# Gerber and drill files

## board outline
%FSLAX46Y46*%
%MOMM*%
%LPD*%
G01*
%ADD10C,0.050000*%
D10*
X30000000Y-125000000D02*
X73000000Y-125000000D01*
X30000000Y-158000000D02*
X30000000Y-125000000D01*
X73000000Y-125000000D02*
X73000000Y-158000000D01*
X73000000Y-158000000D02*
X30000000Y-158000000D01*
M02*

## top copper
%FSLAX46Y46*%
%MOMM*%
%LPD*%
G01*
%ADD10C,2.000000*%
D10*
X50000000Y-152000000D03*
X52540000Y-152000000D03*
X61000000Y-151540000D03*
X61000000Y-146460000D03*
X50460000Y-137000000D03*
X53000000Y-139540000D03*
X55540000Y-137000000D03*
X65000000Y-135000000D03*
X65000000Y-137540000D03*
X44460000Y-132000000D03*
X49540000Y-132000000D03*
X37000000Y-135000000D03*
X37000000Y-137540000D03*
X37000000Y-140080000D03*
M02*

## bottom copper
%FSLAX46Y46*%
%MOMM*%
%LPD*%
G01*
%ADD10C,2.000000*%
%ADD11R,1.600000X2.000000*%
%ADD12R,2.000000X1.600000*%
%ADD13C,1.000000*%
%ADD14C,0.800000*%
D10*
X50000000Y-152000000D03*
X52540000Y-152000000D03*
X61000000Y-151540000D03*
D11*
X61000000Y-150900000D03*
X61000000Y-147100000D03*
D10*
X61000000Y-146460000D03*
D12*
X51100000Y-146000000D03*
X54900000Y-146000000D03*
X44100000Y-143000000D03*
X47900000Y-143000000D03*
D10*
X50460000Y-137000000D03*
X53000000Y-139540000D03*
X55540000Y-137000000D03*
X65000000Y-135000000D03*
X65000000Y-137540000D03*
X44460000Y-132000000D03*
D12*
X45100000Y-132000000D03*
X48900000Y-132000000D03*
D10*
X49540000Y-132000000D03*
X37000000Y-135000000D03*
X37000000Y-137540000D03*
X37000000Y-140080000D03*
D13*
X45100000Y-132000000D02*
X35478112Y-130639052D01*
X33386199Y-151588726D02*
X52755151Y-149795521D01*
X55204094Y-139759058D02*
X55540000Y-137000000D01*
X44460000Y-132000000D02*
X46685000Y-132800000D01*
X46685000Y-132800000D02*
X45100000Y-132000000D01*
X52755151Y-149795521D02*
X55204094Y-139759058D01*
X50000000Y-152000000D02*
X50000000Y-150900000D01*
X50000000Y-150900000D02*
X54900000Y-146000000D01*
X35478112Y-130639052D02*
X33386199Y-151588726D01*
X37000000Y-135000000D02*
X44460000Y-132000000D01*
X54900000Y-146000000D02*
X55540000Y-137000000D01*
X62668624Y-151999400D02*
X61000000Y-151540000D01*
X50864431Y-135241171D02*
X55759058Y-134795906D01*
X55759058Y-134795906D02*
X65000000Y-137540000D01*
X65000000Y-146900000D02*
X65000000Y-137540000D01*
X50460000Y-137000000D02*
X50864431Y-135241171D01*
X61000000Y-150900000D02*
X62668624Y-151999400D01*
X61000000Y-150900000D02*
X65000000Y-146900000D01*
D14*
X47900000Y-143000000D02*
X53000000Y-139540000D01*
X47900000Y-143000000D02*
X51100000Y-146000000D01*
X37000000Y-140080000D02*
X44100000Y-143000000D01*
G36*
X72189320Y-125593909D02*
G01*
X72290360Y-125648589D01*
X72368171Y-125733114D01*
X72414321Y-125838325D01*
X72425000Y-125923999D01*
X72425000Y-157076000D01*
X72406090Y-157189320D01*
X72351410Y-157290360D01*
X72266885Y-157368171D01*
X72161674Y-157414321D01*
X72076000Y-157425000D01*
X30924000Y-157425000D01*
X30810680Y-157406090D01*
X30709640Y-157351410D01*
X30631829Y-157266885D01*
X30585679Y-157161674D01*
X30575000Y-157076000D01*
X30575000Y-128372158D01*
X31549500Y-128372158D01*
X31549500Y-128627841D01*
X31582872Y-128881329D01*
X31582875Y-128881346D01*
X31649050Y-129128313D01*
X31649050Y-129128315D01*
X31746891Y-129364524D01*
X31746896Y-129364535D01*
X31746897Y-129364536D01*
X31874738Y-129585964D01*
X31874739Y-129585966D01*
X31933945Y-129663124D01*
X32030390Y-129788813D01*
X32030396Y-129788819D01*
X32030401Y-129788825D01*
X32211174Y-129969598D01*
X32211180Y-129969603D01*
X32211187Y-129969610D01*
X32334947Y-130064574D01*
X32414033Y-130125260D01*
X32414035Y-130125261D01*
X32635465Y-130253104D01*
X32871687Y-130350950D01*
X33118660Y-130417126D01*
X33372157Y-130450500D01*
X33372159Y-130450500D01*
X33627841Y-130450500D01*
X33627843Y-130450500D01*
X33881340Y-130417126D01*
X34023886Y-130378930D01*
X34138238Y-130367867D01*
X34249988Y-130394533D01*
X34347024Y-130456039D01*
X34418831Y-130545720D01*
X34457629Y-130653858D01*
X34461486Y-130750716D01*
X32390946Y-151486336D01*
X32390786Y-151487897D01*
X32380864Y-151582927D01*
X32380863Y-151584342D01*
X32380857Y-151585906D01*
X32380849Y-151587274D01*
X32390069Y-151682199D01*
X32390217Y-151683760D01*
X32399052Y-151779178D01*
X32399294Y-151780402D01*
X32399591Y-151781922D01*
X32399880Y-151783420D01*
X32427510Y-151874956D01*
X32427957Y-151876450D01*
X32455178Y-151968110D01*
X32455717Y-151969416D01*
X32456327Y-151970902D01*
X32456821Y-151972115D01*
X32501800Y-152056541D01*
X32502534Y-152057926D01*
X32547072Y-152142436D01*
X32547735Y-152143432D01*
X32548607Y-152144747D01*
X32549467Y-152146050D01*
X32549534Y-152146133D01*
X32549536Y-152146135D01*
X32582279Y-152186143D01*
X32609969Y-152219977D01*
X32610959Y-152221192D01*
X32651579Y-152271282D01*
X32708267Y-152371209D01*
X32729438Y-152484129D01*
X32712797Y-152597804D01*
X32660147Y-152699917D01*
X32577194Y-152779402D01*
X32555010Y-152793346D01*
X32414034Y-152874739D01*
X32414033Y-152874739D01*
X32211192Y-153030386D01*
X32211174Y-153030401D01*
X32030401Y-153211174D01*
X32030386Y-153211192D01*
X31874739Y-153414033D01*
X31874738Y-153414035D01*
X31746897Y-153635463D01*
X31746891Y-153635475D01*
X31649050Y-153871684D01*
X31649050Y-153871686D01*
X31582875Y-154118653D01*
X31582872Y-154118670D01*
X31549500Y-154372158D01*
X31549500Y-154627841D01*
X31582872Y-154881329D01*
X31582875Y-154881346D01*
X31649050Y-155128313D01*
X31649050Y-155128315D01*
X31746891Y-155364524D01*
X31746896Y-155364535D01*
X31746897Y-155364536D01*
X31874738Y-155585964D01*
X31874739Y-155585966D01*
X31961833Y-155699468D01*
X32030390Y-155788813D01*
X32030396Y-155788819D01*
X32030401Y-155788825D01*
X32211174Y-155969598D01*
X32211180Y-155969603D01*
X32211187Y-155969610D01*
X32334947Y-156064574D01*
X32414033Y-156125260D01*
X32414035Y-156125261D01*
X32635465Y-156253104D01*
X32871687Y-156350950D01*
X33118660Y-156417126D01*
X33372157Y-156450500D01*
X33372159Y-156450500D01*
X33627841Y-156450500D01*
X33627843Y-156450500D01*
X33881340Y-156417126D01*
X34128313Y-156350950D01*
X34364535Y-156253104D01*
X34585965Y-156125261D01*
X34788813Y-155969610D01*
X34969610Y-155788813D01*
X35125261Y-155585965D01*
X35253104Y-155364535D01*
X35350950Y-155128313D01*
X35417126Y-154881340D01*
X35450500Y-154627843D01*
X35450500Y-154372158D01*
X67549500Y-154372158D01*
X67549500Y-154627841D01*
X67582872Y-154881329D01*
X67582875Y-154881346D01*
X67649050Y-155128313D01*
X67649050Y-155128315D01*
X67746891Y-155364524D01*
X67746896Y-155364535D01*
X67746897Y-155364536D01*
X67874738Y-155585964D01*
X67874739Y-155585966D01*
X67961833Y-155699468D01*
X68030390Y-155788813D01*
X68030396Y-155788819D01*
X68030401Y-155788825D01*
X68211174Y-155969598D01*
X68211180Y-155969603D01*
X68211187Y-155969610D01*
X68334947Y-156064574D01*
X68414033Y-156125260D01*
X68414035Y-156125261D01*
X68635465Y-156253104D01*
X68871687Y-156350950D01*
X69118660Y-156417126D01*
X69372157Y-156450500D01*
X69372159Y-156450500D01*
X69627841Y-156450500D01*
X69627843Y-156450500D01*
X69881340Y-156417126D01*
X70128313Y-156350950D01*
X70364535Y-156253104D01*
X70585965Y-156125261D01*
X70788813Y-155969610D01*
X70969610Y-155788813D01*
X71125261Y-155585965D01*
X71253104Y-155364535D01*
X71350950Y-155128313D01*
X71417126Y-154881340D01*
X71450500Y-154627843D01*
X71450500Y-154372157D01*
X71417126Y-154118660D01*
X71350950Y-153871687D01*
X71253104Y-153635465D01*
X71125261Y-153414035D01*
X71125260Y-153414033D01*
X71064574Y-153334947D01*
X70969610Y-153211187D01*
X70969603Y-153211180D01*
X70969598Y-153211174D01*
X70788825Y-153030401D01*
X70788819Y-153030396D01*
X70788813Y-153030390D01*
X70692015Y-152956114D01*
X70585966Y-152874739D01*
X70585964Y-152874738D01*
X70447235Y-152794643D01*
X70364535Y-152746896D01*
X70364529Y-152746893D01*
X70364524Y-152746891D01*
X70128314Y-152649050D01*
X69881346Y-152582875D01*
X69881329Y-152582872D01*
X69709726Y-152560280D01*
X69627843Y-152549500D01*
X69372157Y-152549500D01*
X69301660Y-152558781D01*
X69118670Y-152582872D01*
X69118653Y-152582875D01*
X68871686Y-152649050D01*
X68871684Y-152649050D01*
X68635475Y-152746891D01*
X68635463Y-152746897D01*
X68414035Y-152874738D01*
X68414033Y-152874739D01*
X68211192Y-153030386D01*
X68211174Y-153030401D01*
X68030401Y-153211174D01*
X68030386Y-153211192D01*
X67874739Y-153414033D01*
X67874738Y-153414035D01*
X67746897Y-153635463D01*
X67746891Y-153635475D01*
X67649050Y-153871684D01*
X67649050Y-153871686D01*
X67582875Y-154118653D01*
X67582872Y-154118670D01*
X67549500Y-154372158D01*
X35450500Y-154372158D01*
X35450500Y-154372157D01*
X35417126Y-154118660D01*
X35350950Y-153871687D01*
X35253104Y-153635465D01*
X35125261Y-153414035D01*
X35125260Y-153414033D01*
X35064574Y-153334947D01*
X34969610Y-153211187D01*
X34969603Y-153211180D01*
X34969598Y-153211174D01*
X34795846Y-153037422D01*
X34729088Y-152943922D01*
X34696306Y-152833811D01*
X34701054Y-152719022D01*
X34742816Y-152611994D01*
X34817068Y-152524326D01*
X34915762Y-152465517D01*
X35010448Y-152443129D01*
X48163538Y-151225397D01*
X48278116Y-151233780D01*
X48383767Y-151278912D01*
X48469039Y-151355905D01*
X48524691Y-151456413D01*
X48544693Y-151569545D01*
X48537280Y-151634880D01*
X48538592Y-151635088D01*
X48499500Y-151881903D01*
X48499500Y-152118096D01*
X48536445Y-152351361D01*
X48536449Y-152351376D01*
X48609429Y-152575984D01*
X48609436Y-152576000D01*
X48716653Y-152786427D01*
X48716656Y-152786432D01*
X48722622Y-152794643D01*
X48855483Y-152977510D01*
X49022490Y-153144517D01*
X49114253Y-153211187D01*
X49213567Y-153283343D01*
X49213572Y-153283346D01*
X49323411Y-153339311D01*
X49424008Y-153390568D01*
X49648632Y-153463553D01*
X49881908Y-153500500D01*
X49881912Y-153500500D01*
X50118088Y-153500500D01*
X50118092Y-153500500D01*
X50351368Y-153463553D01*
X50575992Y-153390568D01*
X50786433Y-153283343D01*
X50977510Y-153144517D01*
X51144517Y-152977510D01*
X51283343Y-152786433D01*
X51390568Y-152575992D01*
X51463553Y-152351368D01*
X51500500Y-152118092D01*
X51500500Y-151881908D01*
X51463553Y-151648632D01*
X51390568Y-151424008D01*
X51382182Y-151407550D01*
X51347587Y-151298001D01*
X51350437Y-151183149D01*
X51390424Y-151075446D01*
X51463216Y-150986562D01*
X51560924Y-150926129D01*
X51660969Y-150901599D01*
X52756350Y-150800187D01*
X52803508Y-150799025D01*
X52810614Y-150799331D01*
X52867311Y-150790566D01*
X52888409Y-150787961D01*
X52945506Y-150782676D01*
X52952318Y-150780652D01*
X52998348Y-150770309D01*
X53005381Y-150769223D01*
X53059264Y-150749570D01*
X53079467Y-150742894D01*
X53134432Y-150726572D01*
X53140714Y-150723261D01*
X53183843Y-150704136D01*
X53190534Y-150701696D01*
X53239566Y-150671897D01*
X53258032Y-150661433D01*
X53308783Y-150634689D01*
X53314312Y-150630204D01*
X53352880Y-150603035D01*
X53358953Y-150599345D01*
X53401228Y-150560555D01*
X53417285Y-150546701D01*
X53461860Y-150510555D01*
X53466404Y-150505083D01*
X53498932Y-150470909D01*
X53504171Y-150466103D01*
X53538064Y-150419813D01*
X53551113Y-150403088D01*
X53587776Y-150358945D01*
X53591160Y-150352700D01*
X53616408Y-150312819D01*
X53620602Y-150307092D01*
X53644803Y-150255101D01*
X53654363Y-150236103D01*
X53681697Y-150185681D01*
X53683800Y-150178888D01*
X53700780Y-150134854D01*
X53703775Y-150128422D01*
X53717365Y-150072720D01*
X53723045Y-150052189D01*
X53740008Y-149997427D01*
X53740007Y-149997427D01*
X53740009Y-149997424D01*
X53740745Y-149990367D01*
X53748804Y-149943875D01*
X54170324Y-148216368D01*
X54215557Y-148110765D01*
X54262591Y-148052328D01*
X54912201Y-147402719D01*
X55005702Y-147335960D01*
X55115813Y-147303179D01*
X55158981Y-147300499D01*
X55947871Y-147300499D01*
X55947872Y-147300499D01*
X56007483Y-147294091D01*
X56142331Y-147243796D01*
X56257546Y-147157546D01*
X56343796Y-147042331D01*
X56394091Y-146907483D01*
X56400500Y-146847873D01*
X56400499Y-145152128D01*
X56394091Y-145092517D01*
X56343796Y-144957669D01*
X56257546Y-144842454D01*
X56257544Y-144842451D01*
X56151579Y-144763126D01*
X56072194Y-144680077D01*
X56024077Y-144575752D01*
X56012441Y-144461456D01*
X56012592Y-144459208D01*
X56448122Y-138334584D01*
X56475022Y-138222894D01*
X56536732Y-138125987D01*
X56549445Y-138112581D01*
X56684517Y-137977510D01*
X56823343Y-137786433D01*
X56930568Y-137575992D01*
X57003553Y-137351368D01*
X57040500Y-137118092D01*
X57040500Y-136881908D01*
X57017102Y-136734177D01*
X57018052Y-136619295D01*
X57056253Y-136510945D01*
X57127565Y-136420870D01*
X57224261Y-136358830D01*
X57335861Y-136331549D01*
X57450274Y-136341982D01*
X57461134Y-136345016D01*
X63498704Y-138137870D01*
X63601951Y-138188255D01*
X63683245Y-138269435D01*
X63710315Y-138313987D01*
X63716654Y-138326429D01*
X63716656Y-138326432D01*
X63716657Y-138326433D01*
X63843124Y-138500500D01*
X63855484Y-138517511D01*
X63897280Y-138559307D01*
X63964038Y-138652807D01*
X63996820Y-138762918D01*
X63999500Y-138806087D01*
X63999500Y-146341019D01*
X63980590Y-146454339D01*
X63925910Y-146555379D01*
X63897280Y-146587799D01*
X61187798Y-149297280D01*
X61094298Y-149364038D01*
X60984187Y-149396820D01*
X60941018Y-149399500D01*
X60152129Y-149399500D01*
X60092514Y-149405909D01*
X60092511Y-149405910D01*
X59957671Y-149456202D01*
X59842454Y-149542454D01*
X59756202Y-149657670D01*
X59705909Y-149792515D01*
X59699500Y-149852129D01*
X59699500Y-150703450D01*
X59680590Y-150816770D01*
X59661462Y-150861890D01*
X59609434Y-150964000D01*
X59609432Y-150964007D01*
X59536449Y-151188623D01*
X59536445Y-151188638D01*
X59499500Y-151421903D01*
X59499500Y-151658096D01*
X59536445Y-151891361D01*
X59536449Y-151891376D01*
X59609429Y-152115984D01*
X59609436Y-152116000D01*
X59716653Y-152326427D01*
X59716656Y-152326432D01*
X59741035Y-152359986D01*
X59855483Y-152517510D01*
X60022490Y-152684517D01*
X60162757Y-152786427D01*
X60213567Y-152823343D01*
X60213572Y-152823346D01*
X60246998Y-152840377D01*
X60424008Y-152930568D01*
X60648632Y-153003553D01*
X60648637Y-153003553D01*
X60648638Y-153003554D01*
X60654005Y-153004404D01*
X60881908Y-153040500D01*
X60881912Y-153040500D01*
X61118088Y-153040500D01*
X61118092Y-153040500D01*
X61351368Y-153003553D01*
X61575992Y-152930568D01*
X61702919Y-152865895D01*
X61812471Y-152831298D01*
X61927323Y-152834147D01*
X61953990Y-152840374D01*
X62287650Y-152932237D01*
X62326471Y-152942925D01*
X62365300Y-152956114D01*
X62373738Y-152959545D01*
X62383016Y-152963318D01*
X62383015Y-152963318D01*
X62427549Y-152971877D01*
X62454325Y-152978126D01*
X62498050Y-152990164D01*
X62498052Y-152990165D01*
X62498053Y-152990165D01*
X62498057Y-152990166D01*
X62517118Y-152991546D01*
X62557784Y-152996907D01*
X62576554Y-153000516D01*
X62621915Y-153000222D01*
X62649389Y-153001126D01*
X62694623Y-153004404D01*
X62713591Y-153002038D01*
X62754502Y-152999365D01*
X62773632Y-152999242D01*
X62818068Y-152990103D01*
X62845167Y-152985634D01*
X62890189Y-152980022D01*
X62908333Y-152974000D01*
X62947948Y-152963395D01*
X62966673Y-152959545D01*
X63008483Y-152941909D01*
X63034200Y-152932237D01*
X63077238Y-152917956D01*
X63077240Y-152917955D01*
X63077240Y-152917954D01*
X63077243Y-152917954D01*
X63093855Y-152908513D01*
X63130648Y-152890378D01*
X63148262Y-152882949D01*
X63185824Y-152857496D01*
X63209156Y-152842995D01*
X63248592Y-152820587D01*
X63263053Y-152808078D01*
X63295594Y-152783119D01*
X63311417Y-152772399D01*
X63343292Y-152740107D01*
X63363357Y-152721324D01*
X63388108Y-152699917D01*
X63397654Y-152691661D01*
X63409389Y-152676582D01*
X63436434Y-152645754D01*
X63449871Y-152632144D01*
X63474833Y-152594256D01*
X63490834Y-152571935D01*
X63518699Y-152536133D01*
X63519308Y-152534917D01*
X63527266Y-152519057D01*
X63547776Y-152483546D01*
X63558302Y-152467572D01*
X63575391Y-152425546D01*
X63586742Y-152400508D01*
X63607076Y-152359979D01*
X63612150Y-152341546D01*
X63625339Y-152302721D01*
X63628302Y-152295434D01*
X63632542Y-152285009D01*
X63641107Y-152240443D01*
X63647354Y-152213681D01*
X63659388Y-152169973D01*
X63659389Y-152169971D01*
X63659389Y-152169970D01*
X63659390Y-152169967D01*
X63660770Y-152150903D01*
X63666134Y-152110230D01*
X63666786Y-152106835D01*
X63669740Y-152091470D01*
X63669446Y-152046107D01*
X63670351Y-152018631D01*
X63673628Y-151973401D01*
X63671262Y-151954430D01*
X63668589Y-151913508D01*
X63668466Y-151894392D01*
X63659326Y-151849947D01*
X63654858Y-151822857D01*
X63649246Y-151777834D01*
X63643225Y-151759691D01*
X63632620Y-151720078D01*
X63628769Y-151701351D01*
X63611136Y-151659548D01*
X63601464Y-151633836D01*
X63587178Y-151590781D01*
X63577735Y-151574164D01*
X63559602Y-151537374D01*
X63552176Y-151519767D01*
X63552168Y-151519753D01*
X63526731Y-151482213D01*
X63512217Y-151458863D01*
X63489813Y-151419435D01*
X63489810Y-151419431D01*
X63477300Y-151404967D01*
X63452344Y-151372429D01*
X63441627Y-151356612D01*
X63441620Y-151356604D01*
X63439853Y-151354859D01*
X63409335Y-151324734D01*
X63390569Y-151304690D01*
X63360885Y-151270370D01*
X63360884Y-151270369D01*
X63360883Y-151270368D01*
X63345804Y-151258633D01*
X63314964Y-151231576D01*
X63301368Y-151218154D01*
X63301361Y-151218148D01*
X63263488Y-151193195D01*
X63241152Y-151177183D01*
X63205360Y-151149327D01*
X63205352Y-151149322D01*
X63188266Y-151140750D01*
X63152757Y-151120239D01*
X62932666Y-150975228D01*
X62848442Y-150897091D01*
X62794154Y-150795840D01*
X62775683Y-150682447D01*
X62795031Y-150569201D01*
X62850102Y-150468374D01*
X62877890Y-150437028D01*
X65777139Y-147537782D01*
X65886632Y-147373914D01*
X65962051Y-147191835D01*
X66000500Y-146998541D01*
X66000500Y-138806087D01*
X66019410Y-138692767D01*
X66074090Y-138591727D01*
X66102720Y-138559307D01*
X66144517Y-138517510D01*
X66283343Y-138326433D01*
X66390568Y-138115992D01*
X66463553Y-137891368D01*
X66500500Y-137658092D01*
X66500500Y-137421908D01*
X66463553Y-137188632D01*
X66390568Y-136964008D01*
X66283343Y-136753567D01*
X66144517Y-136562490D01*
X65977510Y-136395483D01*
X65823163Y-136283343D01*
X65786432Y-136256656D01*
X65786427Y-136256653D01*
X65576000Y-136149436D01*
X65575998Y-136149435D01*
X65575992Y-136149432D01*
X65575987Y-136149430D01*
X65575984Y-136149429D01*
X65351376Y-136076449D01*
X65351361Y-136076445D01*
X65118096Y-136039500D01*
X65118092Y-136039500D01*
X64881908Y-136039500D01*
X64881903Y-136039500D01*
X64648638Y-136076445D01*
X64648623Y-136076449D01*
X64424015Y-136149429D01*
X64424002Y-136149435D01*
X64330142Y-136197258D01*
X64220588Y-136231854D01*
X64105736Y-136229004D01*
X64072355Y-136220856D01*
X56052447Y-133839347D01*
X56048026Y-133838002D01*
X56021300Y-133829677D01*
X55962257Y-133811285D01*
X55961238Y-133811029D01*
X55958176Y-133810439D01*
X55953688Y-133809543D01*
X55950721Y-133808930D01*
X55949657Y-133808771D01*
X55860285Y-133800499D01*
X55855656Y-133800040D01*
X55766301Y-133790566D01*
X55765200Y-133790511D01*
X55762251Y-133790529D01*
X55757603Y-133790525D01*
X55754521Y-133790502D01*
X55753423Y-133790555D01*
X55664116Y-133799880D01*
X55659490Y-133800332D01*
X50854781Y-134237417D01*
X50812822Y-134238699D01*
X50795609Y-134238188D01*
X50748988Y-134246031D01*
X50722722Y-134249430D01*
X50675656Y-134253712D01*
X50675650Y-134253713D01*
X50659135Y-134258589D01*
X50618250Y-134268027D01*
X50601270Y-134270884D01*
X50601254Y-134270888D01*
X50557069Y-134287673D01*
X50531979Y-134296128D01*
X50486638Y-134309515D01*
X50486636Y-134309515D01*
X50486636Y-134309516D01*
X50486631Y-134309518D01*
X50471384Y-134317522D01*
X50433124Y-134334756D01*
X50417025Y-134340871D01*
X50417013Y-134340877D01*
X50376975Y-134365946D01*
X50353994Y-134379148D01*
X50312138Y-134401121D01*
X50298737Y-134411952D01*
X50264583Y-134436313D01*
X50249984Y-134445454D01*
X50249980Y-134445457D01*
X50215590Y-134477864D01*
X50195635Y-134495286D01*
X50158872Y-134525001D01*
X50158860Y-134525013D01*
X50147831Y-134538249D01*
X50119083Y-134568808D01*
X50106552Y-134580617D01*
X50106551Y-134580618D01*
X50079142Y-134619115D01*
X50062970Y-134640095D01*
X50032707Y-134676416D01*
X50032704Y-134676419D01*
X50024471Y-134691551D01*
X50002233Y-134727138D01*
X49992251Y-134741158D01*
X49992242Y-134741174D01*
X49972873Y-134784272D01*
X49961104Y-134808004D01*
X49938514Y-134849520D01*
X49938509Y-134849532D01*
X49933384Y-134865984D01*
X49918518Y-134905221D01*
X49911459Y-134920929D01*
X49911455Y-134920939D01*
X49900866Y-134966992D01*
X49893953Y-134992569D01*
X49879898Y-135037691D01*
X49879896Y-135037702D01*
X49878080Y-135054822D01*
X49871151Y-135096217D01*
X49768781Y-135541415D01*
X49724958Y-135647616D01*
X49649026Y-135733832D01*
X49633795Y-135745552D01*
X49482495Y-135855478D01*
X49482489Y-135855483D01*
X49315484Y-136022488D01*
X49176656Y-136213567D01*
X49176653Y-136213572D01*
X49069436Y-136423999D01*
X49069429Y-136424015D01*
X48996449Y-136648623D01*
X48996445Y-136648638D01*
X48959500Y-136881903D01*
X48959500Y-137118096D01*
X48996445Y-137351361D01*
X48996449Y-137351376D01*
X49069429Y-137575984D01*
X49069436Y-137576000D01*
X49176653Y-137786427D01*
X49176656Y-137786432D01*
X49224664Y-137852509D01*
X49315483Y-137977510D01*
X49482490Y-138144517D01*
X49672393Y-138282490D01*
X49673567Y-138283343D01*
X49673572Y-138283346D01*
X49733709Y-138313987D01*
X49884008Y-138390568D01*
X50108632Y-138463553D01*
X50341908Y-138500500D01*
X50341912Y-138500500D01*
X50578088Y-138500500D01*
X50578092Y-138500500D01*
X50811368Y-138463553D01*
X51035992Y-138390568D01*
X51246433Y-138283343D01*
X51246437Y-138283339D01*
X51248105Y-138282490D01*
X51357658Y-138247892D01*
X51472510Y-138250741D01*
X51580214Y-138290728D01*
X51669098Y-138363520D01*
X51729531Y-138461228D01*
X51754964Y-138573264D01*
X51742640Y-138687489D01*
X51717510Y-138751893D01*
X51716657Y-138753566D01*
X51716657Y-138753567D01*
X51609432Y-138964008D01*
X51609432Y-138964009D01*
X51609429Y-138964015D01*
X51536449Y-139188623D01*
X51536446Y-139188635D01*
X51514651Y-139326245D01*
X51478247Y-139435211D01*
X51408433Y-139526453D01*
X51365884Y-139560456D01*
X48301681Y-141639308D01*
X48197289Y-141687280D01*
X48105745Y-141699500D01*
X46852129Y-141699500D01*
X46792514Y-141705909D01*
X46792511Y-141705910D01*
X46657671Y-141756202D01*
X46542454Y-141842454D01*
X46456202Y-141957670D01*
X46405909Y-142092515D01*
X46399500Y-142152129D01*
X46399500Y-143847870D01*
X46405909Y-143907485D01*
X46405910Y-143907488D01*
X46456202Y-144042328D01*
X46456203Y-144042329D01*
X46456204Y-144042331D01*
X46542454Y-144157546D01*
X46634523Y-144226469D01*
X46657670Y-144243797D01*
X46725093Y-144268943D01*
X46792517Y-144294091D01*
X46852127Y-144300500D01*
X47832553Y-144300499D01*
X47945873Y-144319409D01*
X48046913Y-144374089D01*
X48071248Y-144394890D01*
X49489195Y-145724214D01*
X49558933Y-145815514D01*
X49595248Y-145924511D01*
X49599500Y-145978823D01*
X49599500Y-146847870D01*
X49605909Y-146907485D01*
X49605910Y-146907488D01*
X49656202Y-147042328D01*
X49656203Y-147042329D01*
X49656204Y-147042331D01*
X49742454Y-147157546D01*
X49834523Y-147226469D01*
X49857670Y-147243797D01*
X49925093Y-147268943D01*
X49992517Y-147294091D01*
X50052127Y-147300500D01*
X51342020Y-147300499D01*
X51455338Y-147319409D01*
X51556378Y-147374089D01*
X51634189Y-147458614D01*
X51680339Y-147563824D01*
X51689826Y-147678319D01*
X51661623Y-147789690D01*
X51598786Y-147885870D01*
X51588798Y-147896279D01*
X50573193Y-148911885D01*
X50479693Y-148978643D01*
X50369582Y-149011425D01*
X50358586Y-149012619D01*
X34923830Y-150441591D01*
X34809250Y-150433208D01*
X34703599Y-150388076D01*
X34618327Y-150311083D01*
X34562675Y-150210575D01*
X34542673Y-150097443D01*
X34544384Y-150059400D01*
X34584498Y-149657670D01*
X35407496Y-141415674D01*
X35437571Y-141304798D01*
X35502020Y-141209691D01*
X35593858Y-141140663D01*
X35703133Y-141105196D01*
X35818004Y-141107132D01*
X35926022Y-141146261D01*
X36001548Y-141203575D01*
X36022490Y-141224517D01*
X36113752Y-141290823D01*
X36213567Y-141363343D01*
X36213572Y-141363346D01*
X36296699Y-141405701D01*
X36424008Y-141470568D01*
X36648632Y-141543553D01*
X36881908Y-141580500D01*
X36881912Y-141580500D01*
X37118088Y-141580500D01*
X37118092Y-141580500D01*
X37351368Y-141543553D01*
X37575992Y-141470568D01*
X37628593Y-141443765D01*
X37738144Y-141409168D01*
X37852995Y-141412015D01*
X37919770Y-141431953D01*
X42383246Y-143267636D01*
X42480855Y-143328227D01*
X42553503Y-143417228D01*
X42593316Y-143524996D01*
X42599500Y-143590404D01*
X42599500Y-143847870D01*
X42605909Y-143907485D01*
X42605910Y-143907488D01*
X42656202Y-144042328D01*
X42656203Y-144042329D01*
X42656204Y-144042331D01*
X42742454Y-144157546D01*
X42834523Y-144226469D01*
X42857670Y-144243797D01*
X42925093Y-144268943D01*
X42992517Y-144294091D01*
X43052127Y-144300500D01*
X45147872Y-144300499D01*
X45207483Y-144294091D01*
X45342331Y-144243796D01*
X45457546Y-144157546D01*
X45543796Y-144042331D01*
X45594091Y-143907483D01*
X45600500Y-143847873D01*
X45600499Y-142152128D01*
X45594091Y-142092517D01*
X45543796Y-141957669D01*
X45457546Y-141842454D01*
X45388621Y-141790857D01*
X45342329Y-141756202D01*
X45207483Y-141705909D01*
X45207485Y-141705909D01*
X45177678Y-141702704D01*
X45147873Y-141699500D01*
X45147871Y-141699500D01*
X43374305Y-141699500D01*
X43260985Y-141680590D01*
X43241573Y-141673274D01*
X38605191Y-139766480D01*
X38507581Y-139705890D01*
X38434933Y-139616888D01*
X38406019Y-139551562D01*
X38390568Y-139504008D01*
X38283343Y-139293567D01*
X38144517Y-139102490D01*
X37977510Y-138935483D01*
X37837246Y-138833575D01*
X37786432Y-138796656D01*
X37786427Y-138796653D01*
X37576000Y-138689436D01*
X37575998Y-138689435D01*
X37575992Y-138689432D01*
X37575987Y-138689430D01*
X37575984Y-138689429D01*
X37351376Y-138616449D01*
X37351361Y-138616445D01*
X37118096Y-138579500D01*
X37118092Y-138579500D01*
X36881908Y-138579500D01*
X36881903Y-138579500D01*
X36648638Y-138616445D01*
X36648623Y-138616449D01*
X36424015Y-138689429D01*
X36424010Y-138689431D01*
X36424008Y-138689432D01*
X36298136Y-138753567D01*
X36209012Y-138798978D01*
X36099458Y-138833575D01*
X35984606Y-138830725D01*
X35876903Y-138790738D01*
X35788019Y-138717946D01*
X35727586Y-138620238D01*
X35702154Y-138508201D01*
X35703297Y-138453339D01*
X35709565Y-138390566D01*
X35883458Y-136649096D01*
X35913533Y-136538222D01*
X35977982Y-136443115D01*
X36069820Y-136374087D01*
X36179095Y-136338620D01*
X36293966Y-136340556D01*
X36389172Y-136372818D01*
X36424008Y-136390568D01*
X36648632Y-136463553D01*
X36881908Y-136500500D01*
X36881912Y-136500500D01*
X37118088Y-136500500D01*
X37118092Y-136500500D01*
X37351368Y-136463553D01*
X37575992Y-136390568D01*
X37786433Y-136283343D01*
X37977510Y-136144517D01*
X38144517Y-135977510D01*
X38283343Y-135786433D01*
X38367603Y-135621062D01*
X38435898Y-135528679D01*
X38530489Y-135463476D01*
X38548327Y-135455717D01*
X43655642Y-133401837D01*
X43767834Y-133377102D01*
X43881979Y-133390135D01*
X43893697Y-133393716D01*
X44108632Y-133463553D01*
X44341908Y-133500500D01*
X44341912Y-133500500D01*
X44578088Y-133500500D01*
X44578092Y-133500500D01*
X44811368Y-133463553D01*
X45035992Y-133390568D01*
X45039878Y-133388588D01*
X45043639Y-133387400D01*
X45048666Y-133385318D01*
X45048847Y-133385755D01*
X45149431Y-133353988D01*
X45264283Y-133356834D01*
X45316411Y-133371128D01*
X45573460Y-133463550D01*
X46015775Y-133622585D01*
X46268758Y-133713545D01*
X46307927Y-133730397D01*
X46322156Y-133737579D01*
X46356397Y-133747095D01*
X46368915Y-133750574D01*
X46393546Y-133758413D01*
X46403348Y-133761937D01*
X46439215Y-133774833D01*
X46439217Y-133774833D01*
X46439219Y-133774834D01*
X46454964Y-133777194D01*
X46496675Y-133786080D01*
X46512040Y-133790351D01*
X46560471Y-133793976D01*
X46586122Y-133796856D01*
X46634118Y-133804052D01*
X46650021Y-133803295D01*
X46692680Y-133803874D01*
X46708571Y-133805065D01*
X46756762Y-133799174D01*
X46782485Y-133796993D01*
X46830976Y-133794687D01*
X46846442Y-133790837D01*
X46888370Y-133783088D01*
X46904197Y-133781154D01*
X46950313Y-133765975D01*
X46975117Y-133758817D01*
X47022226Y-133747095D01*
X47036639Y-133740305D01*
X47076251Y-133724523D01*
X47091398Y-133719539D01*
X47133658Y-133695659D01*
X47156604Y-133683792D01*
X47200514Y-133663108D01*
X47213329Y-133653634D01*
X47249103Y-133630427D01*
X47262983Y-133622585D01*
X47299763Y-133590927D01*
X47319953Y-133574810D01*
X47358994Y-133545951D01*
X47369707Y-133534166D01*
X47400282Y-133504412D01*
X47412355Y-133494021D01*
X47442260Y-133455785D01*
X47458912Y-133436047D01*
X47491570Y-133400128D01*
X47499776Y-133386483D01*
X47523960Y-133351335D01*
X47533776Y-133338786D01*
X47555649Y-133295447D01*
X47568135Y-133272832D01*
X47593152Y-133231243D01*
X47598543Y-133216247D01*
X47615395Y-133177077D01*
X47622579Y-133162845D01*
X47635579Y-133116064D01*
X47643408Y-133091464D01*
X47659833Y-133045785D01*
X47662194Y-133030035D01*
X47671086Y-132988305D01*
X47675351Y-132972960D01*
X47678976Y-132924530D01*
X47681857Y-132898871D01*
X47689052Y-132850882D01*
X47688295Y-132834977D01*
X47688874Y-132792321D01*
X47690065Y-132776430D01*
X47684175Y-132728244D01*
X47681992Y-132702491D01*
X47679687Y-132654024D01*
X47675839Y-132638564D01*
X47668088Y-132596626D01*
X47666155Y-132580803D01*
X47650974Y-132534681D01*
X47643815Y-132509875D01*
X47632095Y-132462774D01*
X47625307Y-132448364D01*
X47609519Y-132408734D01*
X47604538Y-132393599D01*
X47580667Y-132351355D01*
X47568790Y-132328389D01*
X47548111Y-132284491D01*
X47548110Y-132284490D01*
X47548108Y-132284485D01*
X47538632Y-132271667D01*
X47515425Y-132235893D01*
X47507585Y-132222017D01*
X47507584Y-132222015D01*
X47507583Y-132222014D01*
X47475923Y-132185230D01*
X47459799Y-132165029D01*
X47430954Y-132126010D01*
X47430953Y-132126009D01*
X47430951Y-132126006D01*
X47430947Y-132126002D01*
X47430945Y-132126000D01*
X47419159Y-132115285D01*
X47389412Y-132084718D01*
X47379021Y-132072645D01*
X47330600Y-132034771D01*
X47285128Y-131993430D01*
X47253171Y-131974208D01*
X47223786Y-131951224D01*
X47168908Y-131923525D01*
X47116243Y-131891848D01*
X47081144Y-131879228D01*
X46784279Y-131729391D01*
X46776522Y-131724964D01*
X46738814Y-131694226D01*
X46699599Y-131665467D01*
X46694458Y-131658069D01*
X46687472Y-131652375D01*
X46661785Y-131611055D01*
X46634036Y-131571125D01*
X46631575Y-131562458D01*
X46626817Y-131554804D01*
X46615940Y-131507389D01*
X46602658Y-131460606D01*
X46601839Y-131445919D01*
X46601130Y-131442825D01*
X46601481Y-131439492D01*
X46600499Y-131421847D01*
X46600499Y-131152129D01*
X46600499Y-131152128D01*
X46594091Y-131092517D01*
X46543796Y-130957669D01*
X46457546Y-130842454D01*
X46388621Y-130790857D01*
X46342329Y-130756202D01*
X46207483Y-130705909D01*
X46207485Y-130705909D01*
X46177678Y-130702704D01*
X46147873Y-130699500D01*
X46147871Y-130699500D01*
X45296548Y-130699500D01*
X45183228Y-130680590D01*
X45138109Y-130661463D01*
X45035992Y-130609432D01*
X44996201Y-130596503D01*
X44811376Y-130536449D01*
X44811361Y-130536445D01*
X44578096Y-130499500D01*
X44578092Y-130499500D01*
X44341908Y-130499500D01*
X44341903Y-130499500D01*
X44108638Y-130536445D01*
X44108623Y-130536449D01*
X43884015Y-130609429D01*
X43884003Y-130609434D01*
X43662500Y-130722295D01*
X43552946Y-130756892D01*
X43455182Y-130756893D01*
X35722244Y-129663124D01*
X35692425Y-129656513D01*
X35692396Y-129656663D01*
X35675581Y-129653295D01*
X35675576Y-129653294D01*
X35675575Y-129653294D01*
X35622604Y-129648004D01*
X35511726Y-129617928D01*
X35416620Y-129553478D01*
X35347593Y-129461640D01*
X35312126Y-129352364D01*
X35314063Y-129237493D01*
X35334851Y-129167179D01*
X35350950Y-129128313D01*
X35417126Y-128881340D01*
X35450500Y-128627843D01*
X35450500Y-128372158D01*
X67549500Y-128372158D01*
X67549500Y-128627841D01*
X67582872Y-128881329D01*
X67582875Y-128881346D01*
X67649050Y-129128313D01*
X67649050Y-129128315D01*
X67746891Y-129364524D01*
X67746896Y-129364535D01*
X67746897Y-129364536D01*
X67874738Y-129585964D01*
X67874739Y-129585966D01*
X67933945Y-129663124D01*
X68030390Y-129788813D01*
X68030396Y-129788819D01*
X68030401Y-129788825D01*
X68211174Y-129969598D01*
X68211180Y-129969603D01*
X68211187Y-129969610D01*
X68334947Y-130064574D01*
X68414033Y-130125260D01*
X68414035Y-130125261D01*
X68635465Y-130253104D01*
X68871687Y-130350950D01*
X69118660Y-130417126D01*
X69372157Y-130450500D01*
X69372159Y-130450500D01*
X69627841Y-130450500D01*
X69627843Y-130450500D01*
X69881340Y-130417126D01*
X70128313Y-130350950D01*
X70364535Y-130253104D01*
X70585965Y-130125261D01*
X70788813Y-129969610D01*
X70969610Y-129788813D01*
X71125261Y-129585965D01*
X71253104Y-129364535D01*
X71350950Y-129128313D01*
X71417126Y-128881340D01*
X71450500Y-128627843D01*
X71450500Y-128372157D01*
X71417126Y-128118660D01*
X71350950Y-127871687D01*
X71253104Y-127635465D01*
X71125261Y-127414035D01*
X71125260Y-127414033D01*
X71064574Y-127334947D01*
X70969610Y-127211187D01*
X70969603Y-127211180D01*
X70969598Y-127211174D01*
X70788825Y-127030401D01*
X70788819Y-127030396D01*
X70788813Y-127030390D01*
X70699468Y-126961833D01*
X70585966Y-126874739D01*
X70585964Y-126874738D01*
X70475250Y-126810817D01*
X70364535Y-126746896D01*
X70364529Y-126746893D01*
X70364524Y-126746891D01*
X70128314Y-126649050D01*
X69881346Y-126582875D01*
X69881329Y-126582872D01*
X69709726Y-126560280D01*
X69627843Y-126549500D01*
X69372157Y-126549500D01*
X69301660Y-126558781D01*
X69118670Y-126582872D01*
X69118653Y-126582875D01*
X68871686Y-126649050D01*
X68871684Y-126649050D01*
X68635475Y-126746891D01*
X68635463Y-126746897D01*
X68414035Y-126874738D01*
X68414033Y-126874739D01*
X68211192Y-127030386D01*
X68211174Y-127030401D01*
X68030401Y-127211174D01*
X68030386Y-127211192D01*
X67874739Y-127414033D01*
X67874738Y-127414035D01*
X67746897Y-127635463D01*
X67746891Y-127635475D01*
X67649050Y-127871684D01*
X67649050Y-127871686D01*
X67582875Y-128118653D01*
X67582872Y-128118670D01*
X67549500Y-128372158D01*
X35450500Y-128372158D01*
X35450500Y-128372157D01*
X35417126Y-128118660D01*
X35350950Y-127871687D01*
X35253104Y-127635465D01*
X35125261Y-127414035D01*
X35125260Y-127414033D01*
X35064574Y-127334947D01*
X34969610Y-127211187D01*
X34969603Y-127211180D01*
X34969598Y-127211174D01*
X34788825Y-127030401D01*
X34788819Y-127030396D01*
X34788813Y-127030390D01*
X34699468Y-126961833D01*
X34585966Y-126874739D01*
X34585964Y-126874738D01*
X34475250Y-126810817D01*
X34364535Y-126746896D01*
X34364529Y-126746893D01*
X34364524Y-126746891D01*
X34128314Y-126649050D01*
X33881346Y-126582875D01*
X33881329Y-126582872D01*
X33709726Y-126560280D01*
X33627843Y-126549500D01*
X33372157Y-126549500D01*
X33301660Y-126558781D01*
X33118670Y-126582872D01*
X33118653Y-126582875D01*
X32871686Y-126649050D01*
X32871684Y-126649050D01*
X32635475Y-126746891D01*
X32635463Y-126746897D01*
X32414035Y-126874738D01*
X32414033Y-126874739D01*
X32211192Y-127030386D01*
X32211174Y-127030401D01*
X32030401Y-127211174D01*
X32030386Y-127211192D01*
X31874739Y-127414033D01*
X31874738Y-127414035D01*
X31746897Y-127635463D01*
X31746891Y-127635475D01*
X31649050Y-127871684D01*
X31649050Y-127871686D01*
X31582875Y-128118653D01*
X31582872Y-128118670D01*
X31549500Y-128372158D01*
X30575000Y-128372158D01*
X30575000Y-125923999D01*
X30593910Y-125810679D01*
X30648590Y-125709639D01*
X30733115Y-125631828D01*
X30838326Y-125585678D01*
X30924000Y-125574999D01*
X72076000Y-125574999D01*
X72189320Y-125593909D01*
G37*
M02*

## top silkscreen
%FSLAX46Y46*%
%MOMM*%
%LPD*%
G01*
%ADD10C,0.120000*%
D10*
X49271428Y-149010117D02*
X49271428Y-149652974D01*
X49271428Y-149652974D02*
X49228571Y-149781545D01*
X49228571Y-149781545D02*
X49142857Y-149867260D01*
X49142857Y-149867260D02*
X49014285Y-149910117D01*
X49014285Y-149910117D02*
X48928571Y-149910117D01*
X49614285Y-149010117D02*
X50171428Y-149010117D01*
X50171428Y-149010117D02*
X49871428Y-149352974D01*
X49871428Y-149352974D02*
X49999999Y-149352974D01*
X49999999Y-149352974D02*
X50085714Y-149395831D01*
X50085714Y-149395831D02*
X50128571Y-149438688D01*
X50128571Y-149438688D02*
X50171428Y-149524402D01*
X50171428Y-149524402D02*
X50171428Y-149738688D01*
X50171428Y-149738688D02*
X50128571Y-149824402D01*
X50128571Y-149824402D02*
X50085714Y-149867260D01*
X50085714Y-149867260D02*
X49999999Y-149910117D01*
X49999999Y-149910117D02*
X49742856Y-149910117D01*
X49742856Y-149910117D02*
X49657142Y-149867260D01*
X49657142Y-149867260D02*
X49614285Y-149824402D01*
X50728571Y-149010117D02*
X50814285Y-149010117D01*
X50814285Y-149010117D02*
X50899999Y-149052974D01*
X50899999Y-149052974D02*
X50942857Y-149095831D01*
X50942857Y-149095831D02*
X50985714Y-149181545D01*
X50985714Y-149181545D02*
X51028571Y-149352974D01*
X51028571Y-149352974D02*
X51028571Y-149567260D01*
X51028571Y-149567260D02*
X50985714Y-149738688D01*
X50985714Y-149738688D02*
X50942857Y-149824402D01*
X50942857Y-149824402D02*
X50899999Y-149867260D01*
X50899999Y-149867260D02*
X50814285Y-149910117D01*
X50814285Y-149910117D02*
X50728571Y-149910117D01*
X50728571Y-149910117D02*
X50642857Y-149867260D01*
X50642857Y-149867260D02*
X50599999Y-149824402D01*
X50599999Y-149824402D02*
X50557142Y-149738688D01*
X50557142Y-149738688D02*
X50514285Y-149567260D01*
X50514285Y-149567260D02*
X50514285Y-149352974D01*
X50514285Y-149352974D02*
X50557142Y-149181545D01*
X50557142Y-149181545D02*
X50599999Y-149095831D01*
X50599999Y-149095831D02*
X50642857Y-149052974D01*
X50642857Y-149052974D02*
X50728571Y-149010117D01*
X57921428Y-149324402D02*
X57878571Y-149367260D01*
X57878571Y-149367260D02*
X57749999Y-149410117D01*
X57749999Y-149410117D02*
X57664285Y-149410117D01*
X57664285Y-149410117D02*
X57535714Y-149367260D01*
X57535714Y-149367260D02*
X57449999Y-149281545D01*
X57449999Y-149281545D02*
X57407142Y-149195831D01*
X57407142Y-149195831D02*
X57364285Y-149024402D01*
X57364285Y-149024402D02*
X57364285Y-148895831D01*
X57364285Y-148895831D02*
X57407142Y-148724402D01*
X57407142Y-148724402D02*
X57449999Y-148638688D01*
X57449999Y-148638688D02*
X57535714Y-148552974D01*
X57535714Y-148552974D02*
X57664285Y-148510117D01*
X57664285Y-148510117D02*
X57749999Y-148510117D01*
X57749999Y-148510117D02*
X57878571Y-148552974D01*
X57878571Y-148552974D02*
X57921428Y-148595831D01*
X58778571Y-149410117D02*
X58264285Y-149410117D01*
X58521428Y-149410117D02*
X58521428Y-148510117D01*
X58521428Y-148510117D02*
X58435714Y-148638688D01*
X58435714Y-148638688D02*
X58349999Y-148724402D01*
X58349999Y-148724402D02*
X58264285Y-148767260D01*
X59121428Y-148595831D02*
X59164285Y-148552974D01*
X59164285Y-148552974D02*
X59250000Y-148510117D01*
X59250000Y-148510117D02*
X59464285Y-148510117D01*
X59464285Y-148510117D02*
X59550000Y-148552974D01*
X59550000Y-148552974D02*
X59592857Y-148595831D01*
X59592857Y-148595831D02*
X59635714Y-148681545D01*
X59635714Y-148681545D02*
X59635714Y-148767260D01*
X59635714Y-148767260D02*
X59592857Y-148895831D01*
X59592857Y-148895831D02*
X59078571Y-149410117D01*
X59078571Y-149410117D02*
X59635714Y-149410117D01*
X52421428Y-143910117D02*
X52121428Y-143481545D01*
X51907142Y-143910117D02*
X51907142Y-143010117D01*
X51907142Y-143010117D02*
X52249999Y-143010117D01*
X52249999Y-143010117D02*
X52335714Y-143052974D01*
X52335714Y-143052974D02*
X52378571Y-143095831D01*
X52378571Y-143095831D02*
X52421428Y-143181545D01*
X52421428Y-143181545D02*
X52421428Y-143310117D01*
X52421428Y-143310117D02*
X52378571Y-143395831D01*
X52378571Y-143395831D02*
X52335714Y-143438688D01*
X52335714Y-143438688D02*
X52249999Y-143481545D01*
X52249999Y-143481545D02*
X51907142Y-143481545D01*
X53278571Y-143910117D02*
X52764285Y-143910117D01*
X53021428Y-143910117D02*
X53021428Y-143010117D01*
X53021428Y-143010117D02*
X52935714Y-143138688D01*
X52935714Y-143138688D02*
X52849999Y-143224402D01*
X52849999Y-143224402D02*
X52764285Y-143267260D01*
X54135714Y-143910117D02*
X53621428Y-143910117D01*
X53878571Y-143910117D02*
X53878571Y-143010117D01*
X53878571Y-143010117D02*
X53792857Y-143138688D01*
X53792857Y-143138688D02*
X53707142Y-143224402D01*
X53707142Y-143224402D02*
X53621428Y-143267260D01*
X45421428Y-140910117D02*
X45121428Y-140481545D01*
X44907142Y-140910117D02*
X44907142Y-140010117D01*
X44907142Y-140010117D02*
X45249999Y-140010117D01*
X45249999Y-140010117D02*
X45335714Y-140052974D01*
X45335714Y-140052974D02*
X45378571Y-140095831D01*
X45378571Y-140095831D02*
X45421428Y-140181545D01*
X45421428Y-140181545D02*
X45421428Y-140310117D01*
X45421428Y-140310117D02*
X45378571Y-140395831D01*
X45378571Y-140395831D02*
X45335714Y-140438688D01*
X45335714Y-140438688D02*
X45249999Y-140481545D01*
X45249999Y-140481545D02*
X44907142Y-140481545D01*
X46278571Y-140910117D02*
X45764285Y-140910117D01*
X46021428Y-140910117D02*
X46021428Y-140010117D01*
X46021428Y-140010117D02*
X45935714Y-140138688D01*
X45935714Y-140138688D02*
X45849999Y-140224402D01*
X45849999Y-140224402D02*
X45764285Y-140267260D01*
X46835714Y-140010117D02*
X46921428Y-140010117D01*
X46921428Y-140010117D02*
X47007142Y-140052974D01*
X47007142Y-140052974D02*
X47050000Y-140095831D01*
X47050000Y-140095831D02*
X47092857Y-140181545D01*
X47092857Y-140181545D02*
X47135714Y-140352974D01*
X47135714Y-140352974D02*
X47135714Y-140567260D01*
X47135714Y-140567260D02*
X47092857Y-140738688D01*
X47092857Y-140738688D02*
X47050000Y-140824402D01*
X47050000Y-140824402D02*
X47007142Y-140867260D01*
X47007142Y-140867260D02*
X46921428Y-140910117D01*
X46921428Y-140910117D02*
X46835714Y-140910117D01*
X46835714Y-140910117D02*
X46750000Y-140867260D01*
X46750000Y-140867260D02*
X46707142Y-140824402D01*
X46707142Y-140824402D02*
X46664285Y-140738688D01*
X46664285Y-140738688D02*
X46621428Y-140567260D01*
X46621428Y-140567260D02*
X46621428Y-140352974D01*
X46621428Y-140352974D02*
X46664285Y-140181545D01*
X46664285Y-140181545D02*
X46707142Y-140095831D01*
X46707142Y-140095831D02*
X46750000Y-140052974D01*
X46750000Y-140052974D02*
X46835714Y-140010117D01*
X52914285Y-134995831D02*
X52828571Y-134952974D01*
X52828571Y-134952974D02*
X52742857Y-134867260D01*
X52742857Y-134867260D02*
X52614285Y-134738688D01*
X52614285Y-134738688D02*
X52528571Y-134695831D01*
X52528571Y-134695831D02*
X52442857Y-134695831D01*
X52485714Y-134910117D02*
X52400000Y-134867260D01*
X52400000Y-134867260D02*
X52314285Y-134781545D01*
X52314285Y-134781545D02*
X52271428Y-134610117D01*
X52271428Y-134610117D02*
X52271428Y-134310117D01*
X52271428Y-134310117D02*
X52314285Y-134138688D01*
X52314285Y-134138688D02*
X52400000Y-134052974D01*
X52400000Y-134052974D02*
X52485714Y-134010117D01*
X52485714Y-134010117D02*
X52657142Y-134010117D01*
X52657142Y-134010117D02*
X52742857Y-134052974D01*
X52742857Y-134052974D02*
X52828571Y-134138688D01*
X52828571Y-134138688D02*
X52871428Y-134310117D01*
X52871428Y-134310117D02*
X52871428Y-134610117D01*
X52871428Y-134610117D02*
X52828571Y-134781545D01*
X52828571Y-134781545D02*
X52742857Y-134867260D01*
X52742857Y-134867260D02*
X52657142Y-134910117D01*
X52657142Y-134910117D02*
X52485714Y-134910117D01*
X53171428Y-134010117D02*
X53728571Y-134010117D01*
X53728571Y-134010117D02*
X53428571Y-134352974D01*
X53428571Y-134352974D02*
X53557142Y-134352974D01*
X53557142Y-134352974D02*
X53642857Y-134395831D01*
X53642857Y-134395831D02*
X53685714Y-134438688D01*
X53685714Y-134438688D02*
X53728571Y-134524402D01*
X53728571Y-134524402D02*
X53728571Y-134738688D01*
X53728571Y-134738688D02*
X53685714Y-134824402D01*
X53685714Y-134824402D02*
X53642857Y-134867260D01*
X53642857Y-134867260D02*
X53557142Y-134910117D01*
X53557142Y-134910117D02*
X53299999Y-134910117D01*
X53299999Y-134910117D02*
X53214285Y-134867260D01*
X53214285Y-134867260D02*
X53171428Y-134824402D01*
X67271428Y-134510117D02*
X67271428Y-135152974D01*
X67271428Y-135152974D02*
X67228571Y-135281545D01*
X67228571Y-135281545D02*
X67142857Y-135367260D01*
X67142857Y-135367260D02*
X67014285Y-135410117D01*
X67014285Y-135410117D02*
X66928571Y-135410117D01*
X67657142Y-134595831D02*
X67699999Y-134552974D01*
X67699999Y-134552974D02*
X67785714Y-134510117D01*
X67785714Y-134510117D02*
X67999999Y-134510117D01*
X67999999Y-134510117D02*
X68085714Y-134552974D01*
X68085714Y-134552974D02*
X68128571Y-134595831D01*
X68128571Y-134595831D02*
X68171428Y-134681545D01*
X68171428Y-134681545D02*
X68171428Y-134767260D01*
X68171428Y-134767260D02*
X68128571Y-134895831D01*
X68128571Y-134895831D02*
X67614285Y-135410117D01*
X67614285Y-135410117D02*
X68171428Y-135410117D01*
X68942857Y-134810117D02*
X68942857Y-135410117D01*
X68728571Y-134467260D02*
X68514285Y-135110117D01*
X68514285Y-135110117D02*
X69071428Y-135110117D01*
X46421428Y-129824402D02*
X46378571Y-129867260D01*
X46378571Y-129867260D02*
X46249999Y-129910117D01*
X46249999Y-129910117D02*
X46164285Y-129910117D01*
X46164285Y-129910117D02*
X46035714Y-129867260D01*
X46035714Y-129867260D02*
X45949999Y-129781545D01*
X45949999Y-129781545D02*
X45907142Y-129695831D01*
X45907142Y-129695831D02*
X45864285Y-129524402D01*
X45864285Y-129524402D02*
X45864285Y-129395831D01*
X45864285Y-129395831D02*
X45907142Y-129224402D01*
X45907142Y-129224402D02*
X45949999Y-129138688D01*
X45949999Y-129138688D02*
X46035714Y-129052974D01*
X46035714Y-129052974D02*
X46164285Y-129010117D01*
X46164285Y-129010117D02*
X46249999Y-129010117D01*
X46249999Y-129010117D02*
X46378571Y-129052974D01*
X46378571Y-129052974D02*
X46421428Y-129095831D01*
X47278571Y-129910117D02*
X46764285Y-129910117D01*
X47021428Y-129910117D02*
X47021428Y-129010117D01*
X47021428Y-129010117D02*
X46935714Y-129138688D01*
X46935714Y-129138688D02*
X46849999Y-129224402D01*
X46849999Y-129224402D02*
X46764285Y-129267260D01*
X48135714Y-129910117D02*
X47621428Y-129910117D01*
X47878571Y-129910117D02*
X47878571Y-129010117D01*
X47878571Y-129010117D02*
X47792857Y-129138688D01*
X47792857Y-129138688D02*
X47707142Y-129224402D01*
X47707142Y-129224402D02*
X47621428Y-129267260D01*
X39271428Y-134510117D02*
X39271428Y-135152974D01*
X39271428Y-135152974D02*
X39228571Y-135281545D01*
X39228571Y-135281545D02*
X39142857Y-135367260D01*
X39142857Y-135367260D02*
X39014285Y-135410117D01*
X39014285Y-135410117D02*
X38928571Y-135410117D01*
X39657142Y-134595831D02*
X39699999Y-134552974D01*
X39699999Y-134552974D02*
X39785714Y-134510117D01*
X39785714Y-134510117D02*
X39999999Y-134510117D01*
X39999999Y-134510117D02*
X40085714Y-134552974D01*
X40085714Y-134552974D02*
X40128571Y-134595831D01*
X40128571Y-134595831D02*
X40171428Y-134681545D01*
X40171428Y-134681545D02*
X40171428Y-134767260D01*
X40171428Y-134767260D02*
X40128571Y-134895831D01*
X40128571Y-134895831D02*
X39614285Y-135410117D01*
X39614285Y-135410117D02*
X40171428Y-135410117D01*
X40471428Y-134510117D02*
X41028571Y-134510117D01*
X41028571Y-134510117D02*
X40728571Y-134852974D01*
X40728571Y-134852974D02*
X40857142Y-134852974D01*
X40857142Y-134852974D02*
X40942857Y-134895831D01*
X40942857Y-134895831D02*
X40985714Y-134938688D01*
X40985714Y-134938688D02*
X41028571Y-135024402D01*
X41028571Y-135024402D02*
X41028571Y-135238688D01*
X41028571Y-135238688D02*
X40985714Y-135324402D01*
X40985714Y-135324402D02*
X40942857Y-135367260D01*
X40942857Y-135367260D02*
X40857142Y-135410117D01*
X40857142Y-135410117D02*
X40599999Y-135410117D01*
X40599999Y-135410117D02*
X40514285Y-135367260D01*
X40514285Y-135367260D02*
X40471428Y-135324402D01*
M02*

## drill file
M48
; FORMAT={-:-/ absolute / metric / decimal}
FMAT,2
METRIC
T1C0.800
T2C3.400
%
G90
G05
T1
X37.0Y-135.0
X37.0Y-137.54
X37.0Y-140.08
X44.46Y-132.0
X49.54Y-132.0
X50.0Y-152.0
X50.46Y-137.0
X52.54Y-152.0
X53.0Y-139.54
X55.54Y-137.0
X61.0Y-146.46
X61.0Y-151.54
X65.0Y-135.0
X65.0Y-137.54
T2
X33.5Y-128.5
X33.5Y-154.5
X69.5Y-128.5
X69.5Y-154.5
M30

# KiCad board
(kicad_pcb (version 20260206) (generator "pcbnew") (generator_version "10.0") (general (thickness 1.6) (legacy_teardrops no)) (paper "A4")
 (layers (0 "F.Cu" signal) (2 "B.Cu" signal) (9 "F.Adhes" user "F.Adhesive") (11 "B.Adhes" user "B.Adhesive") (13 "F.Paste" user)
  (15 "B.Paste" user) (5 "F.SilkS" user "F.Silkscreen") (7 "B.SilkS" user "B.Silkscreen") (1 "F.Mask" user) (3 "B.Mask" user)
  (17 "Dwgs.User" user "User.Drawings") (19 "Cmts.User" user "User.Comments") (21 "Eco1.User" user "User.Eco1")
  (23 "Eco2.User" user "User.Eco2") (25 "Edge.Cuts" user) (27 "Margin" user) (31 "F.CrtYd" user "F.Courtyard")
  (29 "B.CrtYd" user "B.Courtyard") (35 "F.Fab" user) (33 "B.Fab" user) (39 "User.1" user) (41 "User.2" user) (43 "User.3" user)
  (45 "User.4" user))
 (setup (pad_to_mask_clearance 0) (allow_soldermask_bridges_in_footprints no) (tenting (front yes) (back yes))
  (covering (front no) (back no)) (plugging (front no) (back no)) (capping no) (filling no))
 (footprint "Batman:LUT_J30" (layer "F.Cu") (at 50 152)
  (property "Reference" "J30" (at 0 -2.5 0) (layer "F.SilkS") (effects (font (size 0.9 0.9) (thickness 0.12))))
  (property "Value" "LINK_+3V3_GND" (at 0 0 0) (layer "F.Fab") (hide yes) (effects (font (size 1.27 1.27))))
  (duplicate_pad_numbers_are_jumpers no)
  (pad "1" thru_hole circle (at 0 0) (size 2 2) (drill 0.8) (layers "*.Cu") (remove_unused_layers no) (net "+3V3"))
  (pad "2" thru_hole circle (at 2.54 0) (size 2 2) (drill 0.8) (layers "*.Cu") (remove_unused_layers no) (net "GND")))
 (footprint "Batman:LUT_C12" (layer "F.Cu") (at 61 149 90)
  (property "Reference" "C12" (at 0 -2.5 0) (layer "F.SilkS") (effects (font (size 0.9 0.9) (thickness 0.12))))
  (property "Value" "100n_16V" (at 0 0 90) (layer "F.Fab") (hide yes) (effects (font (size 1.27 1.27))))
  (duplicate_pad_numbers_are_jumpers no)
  (pad "1" thru_hole circle (at -2.54 0 90) (size 2 2) (drill 0.8) (layers "*.Cu") (remove_unused_layers no) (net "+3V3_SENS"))
  (pad "1" smd rect (at -1.9 0 90) (size 2 1.6) (layers "B.Cu") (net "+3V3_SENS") (thermal_bridge_angle 45))
  (pad "2" smd rect (at 1.9 0 90) (size 2 1.6) (layers "B.Cu") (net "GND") (thermal_bridge_angle 45))
  (pad "2" thru_hole circle (at 2.54 0 90) (size 2 2) (drill 0.8) (layers "*.Cu") (remove_unused_layers no) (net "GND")))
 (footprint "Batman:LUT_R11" (layer "F.Cu") (at 53 146)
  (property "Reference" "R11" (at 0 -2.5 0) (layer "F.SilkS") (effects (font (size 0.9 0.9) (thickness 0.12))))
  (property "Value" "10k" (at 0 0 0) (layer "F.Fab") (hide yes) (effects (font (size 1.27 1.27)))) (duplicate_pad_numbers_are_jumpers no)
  (pad "1" smd rect (at -1.9 0) (size 2 1.6) (layers "B.Cu") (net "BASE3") (thermal_bridge_angle 45))
  (pad "2" smd rect (at 1.9 0) (size 2 1.6) (layers "B.Cu") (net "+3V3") (thermal_bridge_angle 45)))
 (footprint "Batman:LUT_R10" (layer "F.Cu") (at 46 143)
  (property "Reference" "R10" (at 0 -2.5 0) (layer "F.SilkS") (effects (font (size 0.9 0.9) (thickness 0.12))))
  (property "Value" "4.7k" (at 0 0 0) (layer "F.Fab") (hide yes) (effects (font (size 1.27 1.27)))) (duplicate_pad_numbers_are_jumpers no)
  (pad "1" smd rect (at -1.9 0) (size 2 1.6) (layers "B.Cu") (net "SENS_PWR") (thermal_bridge_angle 45))
  (pad "2" smd rect (at 1.9 0) (size 2 1.6) (layers "B.Cu") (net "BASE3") (thermal_bridge_angle 45)))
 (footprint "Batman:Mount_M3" (layer "F.Cu") (at 69.5 128.5)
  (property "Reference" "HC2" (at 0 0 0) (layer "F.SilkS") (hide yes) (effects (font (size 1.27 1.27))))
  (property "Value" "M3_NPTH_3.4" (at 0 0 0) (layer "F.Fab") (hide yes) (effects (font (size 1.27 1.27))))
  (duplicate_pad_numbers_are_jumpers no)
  (pad "" np_thru_hole circle (at 0 0) (size 3.4 3.4) (drill 3.4) (layers "*.Cu")))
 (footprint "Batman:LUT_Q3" (layer "F.Cu") (at 53 137)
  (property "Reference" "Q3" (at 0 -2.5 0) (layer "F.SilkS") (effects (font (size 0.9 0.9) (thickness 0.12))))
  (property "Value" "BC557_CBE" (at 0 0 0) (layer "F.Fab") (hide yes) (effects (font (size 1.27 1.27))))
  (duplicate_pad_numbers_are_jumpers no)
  (pad "1" thru_hole circle (at -2.54 0) (size 2 2) (drill 0.8) (layers "*.Cu") (remove_unused_layers no) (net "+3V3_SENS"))
  (pad "2" thru_hole circle (at 0 2.54) (size 2 2) (drill 0.8) (layers "*.Cu") (remove_unused_layers no) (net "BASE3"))
  (pad "3" thru_hole circle (at 2.54 0) (size 2 2) (drill 0.8) (layers "*.Cu") (remove_unused_layers no) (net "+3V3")))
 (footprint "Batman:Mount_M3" (layer "F.Cu") (at 69.5 154.5)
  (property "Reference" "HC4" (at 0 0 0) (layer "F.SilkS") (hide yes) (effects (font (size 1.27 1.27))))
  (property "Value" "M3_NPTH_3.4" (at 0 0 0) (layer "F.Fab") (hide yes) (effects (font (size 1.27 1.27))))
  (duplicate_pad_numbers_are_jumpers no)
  (pad "" np_thru_hole circle (at 0 0) (size 3.4 3.4) (drill 3.4) (layers "*.Cu")))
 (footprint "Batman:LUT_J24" (layer "F.Cu") (at 65 135 -90)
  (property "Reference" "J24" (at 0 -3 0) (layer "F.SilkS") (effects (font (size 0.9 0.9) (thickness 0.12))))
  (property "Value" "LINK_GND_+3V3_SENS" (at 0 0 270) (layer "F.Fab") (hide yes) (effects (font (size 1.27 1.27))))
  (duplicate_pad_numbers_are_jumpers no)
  (pad "1" thru_hole circle (at 0 0 270) (size 2 2) (drill 0.8) (layers "*.Cu") (remove_unused_layers no) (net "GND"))
  (pad "2" thru_hole circle (at 2.54 0 270) (size 2 2) (drill 0.8) (layers "*.Cu") (remove_unused_layers no) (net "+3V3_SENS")))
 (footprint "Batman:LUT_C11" (layer "F.Cu") (at 47 132)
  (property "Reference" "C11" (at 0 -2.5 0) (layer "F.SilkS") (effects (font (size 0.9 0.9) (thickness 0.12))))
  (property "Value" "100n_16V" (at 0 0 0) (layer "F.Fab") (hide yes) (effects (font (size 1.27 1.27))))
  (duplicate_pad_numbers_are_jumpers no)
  (pad "1" thru_hole circle (at -2.54 0) (size 2 2) (drill 0.8) (layers "*.Cu") (remove_unused_layers no) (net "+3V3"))
  (pad "1" smd rect (at -1.9 0) (size 2 1.6) (layers "B.Cu") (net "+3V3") (thermal_bridge_angle 45))
  (pad "2" smd rect (at 1.9 0) (size 2 1.6) (layers "B.Cu") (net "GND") (thermal_bridge_angle 45))
  (pad "2" thru_hole circle (at 2.54 0) (size 2 2) (drill 0.8) (layers "*.Cu") (remove_unused_layers no) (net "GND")))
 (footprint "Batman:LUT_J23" (layer "F.Cu") (at 37 135 -90)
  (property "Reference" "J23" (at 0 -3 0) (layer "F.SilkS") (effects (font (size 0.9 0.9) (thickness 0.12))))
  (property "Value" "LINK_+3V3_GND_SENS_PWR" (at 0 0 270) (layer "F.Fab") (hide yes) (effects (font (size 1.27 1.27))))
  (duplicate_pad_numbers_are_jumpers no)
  (pad "1" thru_hole circle (at 0 0 270) (size 2 2) (drill 0.8) (layers "*.Cu") (remove_unused_layers no) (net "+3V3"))
  (pad "2" thru_hole circle (at 2.54 0 270) (size 2 2) (drill 0.8) (layers "*.Cu") (remove_unused_layers no) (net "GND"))
  (pad "3" thru_hole circle (at 5.08 0 270) (size 2 2) (drill 0.8) (layers "*.Cu") (remove_unused_layers no) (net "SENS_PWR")))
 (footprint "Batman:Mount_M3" (layer "F.Cu") (at 33.5 128.5)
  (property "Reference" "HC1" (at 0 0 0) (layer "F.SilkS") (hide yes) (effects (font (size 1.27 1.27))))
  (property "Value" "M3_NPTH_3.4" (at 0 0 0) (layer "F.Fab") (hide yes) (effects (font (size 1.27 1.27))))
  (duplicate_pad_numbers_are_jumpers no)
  (pad "" np_thru_hole circle (at 0 0) (size 3.4 3.4) (drill 3.4) (layers "*.Cu")))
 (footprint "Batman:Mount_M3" (layer "F.Cu") (at 33.5 154.5)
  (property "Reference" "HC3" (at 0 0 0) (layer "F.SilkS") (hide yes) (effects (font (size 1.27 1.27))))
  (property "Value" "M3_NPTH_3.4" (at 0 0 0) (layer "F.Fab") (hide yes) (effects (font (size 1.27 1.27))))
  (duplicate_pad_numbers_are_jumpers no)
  (pad "" np_thru_hole circle (at 0 0) (size 3.4 3.4) (drill 3.4) (layers "*.Cu")))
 (gr_line (start 30 125) (end 73 125) (stroke (width 0.05) (type default)) (layer "Edge.Cuts"))
 (gr_line (start 30 158) (end 30 125) (stroke (width 0.05) (type default)) (layer "Edge.Cuts"))
 (gr_line (start 73 125) (end 73 158) (stroke (width 0.05) (type default)) (layer "Edge.Cuts"))
 (gr_line (start 73 158) (end 30 158) (stroke (width 0.05) (type default)) (layer "Edge.Cuts"))
 (segment (start 45.1 132) (end 35.478112 130.639052) (width 1) (layer "B.Cu") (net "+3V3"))
 (segment (start 33.386199 151.588726) (end 52.755151 149.795521) (width 1) (layer "B.Cu") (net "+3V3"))
 (segment (start 55.204094 139.759058) (end 55.54 137) (width 1) (layer "B.Cu") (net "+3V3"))
 (segment (start 44.46 132) (end 46.685 132.8) (width 1) (layer "B.Cu") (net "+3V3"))
 (segment (start 46.685 132.8) (end 45.1 132) (width 1) (layer "B.Cu") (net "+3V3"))
 (segment (start 52.755151 149.795521) (end 55.204094 139.759058) (width 1) (layer "B.Cu") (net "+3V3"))
 (segment (start 50 152) (end 50 150.9) (width 1) (layer "B.Cu") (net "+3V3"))
 (segment (start 50 150.9) (end 54.9 146) (width 1) (layer "B.Cu") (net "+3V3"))
 (segment (start 35.478112 130.639052) (end 33.386199 151.588726) (width 1) (layer "B.Cu") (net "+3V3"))
 (segment (start 37 135) (end 44.46 132) (width 1) (layer "B.Cu") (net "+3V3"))
 (segment (start 54.9 146) (end 55.54 137) (width 1) (layer "B.Cu") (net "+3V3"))
 (segment (start 62.668624 151.9994) (end 61 151.54) (width 1) (layer "B.Cu") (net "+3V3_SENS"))
 (segment (start 50.864431 135.241171) (end 55.759058 134.795906) (width 1) (layer "B.Cu") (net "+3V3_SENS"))
 (segment (start 55.759058 134.795906) (end 65 137.54) (width 1) (layer "B.Cu") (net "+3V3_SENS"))
 (segment (start 65 146.9) (end 65 137.54) (width 1) (layer "B.Cu") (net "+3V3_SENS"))
 (segment (start 50.46 137) (end 50.864431 135.241171) (width 1) (layer "B.Cu") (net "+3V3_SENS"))
 (segment (start 61 150.9) (end 62.668624 151.9994) (width 1) (layer "B.Cu") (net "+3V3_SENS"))
 (segment (start 61 150.9) (end 65 146.9) (width 1) (layer "B.Cu") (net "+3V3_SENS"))
 (segment (start 47.9 143) (end 53 139.54) (width 0.8) (layer "B.Cu") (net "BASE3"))
 (segment (start 47.9 143) (end 51.1 146) (width 0.8) (layer "B.Cu") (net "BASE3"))
 (segment (start 37 140.08) (end 44.1 143) (width 0.8) (layer "B.Cu") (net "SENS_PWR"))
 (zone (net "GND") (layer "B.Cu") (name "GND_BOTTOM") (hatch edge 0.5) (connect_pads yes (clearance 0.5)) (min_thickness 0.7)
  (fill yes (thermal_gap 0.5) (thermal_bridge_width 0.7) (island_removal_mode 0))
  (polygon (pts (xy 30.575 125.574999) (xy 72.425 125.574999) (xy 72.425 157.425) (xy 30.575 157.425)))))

